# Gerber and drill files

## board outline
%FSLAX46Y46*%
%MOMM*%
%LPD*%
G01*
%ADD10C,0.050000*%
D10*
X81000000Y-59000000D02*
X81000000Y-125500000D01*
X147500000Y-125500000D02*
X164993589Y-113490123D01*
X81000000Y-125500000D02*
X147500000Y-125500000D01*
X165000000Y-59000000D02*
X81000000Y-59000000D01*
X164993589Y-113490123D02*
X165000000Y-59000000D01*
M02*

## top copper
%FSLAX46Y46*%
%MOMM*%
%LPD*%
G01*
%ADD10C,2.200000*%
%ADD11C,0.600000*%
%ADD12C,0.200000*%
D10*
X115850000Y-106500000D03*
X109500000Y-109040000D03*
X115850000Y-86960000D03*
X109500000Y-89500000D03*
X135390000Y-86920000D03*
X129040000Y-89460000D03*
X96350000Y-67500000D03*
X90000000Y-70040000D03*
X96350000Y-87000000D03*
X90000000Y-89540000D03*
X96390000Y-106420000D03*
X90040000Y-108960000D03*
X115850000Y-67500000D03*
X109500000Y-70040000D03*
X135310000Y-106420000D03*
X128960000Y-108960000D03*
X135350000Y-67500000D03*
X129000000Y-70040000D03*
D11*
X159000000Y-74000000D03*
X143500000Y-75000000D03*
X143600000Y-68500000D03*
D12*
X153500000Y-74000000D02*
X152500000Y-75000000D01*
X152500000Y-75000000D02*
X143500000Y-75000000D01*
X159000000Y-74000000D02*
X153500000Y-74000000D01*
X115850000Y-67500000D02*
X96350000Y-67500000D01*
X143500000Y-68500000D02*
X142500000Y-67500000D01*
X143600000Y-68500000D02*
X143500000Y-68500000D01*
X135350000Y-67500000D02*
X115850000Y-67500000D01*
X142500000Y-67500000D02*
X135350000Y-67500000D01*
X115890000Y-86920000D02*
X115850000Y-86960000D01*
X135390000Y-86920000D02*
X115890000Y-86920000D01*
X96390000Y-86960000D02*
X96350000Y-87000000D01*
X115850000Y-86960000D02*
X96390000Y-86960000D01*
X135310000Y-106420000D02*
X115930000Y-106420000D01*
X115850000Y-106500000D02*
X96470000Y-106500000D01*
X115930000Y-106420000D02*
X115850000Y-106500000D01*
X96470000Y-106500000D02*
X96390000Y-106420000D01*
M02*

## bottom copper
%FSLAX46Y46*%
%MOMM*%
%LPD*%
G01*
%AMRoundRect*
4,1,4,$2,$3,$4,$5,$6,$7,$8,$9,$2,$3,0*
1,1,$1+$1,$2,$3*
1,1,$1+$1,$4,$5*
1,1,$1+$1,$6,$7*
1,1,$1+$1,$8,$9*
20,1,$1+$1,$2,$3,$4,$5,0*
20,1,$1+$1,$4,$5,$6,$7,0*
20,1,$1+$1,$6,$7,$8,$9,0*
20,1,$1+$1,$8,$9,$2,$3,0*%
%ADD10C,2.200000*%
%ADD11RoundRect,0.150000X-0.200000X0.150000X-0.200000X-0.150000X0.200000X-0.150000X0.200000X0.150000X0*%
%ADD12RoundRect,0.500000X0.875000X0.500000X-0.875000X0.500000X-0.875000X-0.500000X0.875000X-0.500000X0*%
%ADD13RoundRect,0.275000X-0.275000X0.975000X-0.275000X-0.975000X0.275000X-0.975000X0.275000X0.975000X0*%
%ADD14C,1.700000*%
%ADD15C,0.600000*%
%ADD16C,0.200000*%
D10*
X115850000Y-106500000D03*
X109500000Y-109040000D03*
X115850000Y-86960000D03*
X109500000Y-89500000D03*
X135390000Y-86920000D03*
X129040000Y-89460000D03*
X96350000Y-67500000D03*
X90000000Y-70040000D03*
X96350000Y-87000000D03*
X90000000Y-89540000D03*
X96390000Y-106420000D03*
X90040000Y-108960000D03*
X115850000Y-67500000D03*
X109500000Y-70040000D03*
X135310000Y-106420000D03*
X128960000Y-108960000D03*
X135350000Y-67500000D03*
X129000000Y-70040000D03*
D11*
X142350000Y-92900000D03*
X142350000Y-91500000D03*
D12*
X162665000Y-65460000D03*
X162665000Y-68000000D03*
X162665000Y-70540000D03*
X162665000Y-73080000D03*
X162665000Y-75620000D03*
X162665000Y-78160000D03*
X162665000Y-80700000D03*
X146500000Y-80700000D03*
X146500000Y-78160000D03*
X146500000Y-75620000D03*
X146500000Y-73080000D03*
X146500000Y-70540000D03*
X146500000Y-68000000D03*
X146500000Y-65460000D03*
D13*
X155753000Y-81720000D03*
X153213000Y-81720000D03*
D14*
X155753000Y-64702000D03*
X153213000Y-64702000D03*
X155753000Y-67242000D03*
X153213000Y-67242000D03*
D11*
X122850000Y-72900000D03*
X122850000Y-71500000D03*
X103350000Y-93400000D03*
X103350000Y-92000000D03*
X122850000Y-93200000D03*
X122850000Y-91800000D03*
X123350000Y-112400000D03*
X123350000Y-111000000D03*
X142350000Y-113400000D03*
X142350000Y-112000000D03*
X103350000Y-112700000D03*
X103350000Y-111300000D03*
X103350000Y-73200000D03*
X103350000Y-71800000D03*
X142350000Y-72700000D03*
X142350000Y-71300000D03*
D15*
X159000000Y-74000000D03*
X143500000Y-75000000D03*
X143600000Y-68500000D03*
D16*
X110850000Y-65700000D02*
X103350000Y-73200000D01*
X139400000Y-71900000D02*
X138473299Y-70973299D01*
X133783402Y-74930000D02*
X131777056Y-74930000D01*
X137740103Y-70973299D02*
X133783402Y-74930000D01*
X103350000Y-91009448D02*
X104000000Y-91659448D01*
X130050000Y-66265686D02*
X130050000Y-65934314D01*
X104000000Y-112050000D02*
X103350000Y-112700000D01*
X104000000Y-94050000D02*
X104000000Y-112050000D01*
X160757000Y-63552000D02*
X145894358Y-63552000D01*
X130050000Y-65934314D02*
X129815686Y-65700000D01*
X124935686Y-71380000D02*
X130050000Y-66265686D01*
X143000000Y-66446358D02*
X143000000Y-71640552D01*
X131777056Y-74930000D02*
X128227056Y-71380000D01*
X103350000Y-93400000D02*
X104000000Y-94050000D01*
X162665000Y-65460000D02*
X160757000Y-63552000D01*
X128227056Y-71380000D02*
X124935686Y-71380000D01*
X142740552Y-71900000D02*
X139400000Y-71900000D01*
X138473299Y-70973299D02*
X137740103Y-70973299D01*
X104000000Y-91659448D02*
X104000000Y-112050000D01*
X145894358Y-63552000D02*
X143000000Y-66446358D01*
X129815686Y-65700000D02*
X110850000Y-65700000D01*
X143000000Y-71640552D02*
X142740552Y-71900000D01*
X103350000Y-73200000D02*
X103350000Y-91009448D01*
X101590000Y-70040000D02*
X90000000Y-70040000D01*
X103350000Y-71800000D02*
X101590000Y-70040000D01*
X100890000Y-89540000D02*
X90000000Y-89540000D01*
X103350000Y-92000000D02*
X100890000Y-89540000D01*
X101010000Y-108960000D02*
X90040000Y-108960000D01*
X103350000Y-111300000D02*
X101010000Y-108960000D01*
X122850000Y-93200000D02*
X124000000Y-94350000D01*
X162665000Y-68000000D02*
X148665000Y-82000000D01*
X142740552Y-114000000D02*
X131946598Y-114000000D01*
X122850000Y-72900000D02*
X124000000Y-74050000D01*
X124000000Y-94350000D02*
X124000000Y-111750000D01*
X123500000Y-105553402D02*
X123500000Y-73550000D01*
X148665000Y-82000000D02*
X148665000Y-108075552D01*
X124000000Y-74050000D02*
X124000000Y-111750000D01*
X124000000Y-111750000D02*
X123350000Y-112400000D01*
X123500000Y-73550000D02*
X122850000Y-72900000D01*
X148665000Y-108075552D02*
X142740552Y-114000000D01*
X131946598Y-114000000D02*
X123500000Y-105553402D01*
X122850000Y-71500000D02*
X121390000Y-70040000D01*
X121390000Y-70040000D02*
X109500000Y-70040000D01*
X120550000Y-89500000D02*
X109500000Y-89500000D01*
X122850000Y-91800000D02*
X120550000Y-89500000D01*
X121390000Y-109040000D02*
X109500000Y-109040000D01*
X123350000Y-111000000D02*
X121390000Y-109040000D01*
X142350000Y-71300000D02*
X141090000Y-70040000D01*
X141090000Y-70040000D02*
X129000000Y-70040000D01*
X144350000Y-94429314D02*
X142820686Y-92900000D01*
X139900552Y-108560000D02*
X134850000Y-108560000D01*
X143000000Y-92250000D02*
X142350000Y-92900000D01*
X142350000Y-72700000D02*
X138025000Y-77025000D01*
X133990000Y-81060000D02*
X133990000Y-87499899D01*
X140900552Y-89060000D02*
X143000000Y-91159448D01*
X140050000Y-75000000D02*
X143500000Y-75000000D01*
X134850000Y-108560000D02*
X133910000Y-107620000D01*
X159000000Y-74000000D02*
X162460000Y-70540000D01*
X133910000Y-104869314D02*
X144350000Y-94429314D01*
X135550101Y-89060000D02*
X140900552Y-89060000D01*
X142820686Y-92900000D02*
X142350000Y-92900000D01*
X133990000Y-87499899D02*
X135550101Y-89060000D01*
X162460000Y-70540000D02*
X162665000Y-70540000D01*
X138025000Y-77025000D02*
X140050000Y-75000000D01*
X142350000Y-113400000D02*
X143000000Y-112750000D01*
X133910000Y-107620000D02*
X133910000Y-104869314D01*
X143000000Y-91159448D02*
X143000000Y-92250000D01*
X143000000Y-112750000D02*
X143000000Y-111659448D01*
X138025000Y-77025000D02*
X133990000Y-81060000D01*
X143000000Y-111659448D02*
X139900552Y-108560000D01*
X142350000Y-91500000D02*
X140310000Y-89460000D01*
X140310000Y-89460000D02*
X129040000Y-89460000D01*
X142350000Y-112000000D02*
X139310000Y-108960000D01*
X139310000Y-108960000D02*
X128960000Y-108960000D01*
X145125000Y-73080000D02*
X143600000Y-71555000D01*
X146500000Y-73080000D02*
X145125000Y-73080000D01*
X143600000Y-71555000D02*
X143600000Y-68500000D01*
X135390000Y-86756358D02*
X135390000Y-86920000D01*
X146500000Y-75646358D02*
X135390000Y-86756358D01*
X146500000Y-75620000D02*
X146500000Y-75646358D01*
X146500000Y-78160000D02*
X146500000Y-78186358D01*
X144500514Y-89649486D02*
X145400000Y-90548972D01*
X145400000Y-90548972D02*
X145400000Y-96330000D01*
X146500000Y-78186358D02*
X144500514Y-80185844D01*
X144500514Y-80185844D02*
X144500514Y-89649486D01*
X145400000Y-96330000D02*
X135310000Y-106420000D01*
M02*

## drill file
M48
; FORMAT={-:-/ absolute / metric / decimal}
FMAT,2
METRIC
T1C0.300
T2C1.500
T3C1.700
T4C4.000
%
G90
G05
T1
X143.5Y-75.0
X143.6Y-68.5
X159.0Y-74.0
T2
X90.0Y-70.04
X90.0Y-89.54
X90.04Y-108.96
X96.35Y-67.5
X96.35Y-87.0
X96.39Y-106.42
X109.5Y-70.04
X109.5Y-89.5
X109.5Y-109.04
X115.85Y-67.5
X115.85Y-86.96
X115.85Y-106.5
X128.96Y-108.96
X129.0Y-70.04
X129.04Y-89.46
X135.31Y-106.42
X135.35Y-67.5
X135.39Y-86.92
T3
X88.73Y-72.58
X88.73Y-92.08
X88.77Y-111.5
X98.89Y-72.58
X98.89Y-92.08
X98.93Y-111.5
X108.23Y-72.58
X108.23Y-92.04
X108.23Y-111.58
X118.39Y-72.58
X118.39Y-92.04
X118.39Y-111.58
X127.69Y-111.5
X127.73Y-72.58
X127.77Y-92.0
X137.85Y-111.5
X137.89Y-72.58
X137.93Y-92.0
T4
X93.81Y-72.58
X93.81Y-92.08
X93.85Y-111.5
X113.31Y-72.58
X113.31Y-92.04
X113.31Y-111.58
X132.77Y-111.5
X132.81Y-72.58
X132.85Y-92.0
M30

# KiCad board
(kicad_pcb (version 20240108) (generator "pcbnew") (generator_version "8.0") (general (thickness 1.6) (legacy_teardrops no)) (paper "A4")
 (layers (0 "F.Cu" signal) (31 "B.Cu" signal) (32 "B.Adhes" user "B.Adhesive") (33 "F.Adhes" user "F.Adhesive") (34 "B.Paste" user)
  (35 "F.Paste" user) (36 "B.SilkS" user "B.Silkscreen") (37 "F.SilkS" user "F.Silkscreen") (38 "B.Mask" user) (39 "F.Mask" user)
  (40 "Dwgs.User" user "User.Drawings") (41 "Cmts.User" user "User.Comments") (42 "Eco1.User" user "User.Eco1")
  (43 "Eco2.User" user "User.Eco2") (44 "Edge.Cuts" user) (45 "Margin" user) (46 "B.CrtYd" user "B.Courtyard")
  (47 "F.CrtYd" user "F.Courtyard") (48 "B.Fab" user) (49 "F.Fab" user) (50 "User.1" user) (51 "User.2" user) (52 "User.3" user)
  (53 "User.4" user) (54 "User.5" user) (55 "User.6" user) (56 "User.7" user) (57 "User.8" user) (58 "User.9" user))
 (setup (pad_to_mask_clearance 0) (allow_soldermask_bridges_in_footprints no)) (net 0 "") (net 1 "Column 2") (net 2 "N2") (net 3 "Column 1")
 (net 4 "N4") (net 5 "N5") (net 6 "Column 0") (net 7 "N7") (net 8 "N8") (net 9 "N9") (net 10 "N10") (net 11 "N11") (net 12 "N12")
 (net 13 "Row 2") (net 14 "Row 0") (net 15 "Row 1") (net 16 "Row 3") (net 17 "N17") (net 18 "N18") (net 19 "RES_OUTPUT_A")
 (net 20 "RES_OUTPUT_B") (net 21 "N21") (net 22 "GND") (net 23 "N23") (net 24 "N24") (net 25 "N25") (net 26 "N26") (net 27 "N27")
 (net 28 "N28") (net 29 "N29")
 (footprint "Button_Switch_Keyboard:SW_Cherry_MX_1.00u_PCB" (layer "F.Cu") (at 115.85 106.5)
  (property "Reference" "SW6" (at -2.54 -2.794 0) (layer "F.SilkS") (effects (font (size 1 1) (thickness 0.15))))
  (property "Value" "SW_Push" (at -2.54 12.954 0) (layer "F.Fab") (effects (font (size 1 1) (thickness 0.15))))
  (pad "" np_thru_hole circle (at -7.62 5.08) (size 1.7 1.7) (drill 1.7) (layers "*.Cu" "*.Mask"))
  (pad "" np_thru_hole circle (at -2.54 5.08) (size 4 4) (drill 4) (layers "*.Cu" "*.Mask"))
  (pad "" np_thru_hole circle (at 2.54 5.08) (size 1.7 1.7) (drill 1.7) (layers "*.Cu" "*.Mask"))
  (pad "1" thru_hole circle (at 0 0) (size 2.2 2.2) (drill 1.5) (layers "*.Cu" "*.Mask") (remove_unused_layers no) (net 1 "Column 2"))
  (pad "2" thru_hole circle (at -6.35 2.54) (size 2.2 2.2) (drill 1.5) (layers "*.Cu" "*.Mask") (remove_unused_layers no) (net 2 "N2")))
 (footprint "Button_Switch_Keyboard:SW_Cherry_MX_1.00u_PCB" (layer "F.Cu") (at 115.85 86.96)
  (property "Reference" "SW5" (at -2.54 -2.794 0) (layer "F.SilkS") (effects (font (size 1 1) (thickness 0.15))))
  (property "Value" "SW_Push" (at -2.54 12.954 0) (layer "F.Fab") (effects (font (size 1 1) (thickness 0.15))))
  (pad "" np_thru_hole circle (at -7.62 5.08) (size 1.7 1.7) (drill 1.7) (layers "*.Cu" "*.Mask"))
  (pad "" np_thru_hole circle (at -2.54 5.08) (size 4 4) (drill 4) (layers "*.Cu" "*.Mask"))
  (pad "" np_thru_hole circle (at 2.54 5.08) (size 1.7 1.7) (drill 1.7) (layers "*.Cu" "*.Mask"))
  (pad "1" thru_hole circle (at 0 0) (size 2.2 2.2) (drill 1.5) (layers "*.Cu" "*.Mask") (remove_unused_layers no) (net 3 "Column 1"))
  (pad "2" thru_hole circle (at -6.35 2.54) (size 2.2 2.2) (drill 1.5) (layers "*.Cu" "*.Mask") (remove_unused_layers no) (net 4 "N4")))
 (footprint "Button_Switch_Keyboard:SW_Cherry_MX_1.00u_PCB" (layer "F.Cu") (at 135.39 86.92)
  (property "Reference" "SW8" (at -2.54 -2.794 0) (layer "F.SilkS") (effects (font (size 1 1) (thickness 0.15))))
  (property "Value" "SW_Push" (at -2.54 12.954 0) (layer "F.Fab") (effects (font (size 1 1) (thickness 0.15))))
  (pad "" np_thru_hole circle (at -7.62 5.08) (size 1.7 1.7) (drill 1.7) (layers "*.Cu" "*.Mask"))
  (pad "" np_thru_hole circle (at -2.54 5.08) (size 4 4) (drill 4) (layers "*.Cu" "*.Mask"))
  (pad "" np_thru_hole circle (at 2.54 5.08) (size 1.7 1.7) (drill 1.7) (layers "*.Cu" "*.Mask"))
  (pad "1" thru_hole circle (at 0 0) (size 2.2 2.2) (drill 1.5) (layers "*.Cu" "*.Mask") (remove_unused_layers no) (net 3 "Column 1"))
  (pad "2" thru_hole circle (at -6.35 2.54) (size 2.2 2.2) (drill 1.5) (layers "*.Cu" "*.Mask") (remove_unused_layers no) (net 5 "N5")))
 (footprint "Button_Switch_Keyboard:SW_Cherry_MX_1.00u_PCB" (layer "F.Cu") (at 96.35 67.5)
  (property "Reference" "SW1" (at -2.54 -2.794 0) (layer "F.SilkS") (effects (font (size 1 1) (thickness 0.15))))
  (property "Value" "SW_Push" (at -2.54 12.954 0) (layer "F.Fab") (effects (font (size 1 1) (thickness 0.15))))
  (pad "" np_thru_hole circle (at -7.62 5.08) (size 1.7 1.7) (drill 1.7) (layers "*.Cu" "*.Mask"))
  (pad "" np_thru_hole circle (at -2.54 5.08) (size 4 4) (drill 4) (layers "*.Cu" "*.Mask"))
  (pad "" np_thru_hole circle (at 2.54 5.08) (size 1.7 1.7) (drill 1.7) (layers "*.Cu" "*.Mask"))
  (pad "1" thru_hole circle (at 0 0) (size 2.2 2.2) (drill 1.5) (layers "*.Cu" "*.Mask") (remove_unused_layers no) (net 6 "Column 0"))
  (pad "2" thru_hole circle (at -6.35 2.54) (size 2.2 2.2) (drill 1.5) (layers "*.Cu" "*.Mask") (remove_unused_layers no) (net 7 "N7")))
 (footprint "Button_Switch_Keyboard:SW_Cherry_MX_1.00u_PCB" (layer "F.Cu") (at 96.35 87)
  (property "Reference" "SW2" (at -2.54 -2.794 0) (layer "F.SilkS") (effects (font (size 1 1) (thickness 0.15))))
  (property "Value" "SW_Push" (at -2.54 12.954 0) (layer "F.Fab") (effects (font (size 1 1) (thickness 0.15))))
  (pad "" np_thru_hole circle (at -7.62 5.08) (size 1.7 1.7) (drill 1.7) (layers "*.Cu" "*.Mask"))
  (pad "" np_thru_hole circle (at -2.54 5.08) (size 4 4) (drill 4) (layers "*.Cu" "*.Mask"))
  (pad "" np_thru_hole circle (at 2.54 5.08) (size 1.7 1.7) (drill 1.7) (layers "*.Cu" "*.Mask"))
  (pad "1" thru_hole circle (at 0 0) (size 2.2 2.2) (drill 1.5) (layers "*.Cu" "*.Mask") (remove_unused_layers no) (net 3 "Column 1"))
  (pad "2" thru_hole circle (at -6.35 2.54) (size 2.2 2.2) (drill 1.5) (layers "*.Cu" "*.Mask") (remove_unused_layers no) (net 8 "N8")))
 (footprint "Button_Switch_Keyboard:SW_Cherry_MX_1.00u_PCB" (layer "F.Cu") (at 96.39 106.42)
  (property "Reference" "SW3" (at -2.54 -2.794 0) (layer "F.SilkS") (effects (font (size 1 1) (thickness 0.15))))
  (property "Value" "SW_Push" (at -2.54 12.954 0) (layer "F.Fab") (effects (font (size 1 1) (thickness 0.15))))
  (pad "" np_thru_hole circle (at -7.62 5.08) (size 1.7 1.7) (drill 1.7) (layers "*.Cu" "*.Mask"))
  (pad "" np_thru_hole circle (at -2.54 5.08) (size 4 4) (drill 4) (layers "*.Cu" "*.Mask"))
  (pad "" np_thru_hole circle (at 2.54 5.08) (size 1.7 1.7) (drill 1.7) (layers "*.Cu" "*.Mask"))
  (pad "1" thru_hole circle (at 0 0) (size 2.2 2.2) (drill 1.5) (layers "*.Cu" "*.Mask") (remove_unused_layers no) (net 1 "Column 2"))
  (pad "2" thru_hole circle (at -6.35 2.54) (size 2.2 2.2) (drill 1.5) (layers "*.Cu" "*.Mask") (remove_unused_layers no) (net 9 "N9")))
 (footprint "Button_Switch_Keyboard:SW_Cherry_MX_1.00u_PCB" (layer "F.Cu") (at 115.85 67.5)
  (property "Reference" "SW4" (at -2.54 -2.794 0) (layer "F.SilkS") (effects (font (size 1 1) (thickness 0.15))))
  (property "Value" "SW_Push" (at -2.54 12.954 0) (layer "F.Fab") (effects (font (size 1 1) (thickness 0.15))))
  (pad "" np_thru_hole circle (at -7.62 5.08) (size 1.7 1.7) (drill 1.7) (layers "*.Cu" "*.Mask"))
  (pad "" np_thru_hole circle (at -2.54 5.08) (size 4 4) (drill 4) (layers "*.Cu" "*.Mask"))
  (pad "" np_thru_hole circle (at 2.54 5.08) (size 1.7 1.7) (drill 1.7) (layers "*.Cu" "*.Mask"))
  (pad "1" thru_hole circle (at 0 0) (size 2.2 2.2) (drill 1.5) (layers "*.Cu" "*.Mask") (remove_unused_layers no) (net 6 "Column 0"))
  (pad "2" thru_hole circle (at -6.35 2.54) (size 2.2 2.2) (drill 1.5) (layers "*.Cu" "*.Mask") (remove_unused_layers no) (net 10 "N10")))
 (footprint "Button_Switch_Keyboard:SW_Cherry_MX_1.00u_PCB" (layer "F.Cu") (at 135.31 106.42)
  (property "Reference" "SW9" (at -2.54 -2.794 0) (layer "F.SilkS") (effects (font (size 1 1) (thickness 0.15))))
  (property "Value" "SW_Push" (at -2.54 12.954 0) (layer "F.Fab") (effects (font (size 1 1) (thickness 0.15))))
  (pad "" np_thru_hole circle (at -7.62 5.08) (size 1.7 1.7) (drill 1.7) (layers "*.Cu" "*.Mask"))
  (pad "" np_thru_hole circle (at -2.54 5.08) (size 4 4) (drill 4) (layers "*.Cu" "*.Mask"))
  (pad "" np_thru_hole circle (at 2.54 5.08) (size 1.7 1.7) (drill 1.7) (layers "*.Cu" "*.Mask"))
  (pad "1" thru_hole circle (at 0 0) (size 2.2 2.2) (drill 1.5) (layers "*.Cu" "*.Mask") (remove_unused_layers no) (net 1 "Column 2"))
  (pad "2" thru_hole circle (at -6.35 2.54) (size 2.2 2.2) (drill 1.5) (layers "*.Cu" "*.Mask") (remove_unused_layers no) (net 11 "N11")))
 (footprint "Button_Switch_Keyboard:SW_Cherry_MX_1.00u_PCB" (layer "F.Cu") (at 135.35 67.5)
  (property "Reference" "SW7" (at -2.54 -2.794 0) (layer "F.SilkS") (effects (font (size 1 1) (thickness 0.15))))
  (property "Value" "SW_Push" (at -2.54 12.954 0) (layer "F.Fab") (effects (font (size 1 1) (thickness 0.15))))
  (pad "" np_thru_hole circle (at -7.62 5.08) (size 1.7 1.7) (drill 1.7) (layers "*.Cu" "*.Mask"))
  (pad "" np_thru_hole circle (at -2.54 5.08) (size 4 4) (drill 4) (layers "*.Cu" "*.Mask"))
  (pad "" np_thru_hole circle (at 2.54 5.08) (size 1.7 1.7) (drill 1.7) (layers "*.Cu" "*.Mask"))
  (pad "1" thru_hole circle (at 0 0) (size 2.2 2.2) (drill 1.5) (layers "*.Cu" "*.Mask") (remove_unused_layers no) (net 6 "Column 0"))
  (pad "2" thru_hole circle (at -6.35 2.54) (size 2.2 2.2) (drill 1.5) (layers "*.Cu" "*.Mask") (remove_unused_layers no) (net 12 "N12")))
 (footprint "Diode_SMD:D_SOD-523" (layer "B.Cu") (at 142.35 92.2 90)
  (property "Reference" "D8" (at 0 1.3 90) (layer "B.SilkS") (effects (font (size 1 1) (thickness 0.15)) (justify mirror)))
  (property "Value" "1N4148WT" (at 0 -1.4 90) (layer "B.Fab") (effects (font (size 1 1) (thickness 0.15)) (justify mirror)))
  (pad "1" smd roundrect (at -0.7 0 270) (size 0.6 0.7) (layers "B.Cu" "B.Paste" "B.Mask") (roundrect_rratio 0.25) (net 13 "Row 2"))
  (pad "2" smd roundrect (at 0.7 0 270) (size 0.6 0.7) (layers "B.Cu" "B.Paste" "B.Mask") (roundrect_rratio 0.25) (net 5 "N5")))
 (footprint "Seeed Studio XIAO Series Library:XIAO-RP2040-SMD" (layer "B.Cu") (at 154.665 73.08 180)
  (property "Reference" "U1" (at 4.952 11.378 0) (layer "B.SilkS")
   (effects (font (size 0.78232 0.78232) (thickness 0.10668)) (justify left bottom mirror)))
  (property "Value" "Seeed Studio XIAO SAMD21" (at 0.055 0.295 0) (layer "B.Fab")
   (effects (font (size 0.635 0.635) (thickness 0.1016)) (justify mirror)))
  (pad "1" smd roundrect (at -8 7.62 180) (size 2.75 2) (layers "B.Cu" "B.Paste" "B.Mask") (roundrect_rratio 0.25) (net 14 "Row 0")
   (solder_mask_margin 0.0508) (thermal_bridge_angle 45))
  (pad "2" smd roundrect (at -8 5.08 180) (size 2.75 2) (layers "B.Cu" "B.Paste" "B.Mask") (roundrect_rratio 0.25) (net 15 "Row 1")
   (solder_mask_margin 0.0508) (thermal_bridge_angle 45))
  (pad "3" smd roundrect (at -8 2.54 180) (size 2.75 2) (layers "B.Cu" "B.Paste" "B.Mask") (roundrect_rratio 0.25) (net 13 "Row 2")
   (solder_mask_margin 0.0508) (thermal_bridge_angle 45))
  (pad "4" smd roundrect (at -8 0 180) (size 2.75 2) (layers "B.Cu" "B.Paste" "B.Mask") (roundrect_rratio 0.25) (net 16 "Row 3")
   (solder_mask_margin 0.0508) (thermal_bridge_angle 45))
  (pad "5" smd roundrect (at -8 -2.54 180) (size 2.75 2) (layers "B.Cu" "B.Paste" "B.Mask") (roundrect_rratio 0.25) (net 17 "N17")
   (solder_mask_margin 0.0508) (thermal_bridge_angle 45))
  (pad "6" smd roundrect (at -8 -5.08 180) (size 2.75 2) (layers "B.Cu" "B.Paste" "B.Mask") (roundrect_rratio 0.25) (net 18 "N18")
   (solder_mask_margin 0.0508) (thermal_bridge_angle 45))
  (pad "7" smd roundrect (at -8 -7.62 180) (size 2.75 2) (layers "B.Cu" "B.Paste" "B.Mask") (roundrect_rratio 0.25) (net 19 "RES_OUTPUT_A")
   (solder_mask_margin 0.0508) (thermal_bridge_angle 45))
  (pad "8" smd roundrect (at 8.165 -7.62 180) (size 2.75 2) (layers "B.Cu" "B.Paste" "B.Mask") (roundrect_rratio 0.25)
   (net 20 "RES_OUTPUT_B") (solder_mask_margin 0.0508) (thermal_bridge_angle 45))
  (pad "9" smd roundrect (at 8.165 -5.08 180) (size 2.75 2) (layers "B.Cu" "B.Paste" "B.Mask") (roundrect_rratio 0.25) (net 1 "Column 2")
   (solder_mask_margin 0.0508) (thermal_bridge_angle 45))
  (pad "10" smd roundrect (at 8.165 -2.54 180) (size 2.75 2) (layers "B.Cu" "B.Paste" "B.Mask") (roundrect_rratio 0.25) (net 3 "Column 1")
   (solder_mask_margin 0.0508) (thermal_bridge_angle 45))
  (pad "11" smd roundrect (at 8.165 0 180) (size 2.75 2) (layers "B.Cu" "B.Paste" "B.Mask") (roundrect_rratio 0.25) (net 6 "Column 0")
   (solder_mask_margin 0.0508) (thermal_bridge_angle 45))
  (pad "12" smd roundrect (at 8.165 2.54 180) (size 2.75 2) (layers "B.Cu" "B.Paste" "B.Mask") (roundrect_rratio 0.25) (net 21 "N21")
   (solder_mask_margin 0.0508) (thermal_bridge_angle 45))
  (pad "13" smd roundrect (at 8.165 5.08 180) (size 2.75 2) (layers "B.Cu" "B.Paste" "B.Mask") (roundrect_rratio 0.25) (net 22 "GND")
   (solder_mask_margin 0.0508) (thermal_bridge_angle 45))
  (pad "14" smd roundrect (at 8.165 7.62 180) (size 2.75 2) (layers "B.Cu" "B.Paste" "B.Mask") (roundrect_rratio 0.25) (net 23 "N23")
   (solder_mask_margin 0.0508) (thermal_bridge_angle 45))
  (pad "15" smd roundrect (at -1.088 -8.64 270) (size 2.5 1.1) (layers "B.Cu" "B.Paste" "B.Mask") (roundrect_rratio 0.25) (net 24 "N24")
   (thermal_bridge_angle 45))
  (pad "16" smd roundrect (at 1.452 -8.64 270) (size 2.5 1.1) (layers "B.Cu" "B.Paste" "B.Mask") (roundrect_rratio 0.25) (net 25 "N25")
   (thermal_bridge_angle 45))
  (pad "17" smd circle (at -1.088 8.378 180) (size 1.7 1.7) (layers "B.Cu" "B.Paste" "B.Mask") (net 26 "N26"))
  (pad "18" smd circle (at 1.452 8.378 180) (size 1.7 1.7) (layers "B.Cu" "B.Paste" "B.Mask") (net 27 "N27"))
  (pad "19" smd circle (at -1.088 5.838 180) (size 1.7 1.7) (layers "B.Cu" "B.Paste" "B.Mask") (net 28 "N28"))
  (pad "20" smd circle (at 1.452 5.838 180) (size 1.7 1.7) (layers "B.Cu" "B.Paste" "B.Mask") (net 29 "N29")))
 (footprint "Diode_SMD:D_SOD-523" (layer "B.Cu") (at 122.85 72.2 90)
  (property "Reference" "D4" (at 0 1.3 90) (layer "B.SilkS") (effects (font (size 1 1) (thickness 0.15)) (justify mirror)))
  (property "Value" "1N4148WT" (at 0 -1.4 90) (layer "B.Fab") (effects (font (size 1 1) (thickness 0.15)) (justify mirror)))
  (pad "1" smd roundrect (at -0.7 0 270) (size 0.6 0.7) (layers "B.Cu" "B.Paste" "B.Mask") (roundrect_rratio 0.25) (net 15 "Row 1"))
  (pad "2" smd roundrect (at 0.7 0 270) (size 0.6 0.7) (layers "B.Cu" "B.Paste" "B.Mask") (roundrect_rratio 0.25) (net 10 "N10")))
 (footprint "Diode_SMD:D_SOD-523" (layer "B.Cu") (at 103.35 92.7 90)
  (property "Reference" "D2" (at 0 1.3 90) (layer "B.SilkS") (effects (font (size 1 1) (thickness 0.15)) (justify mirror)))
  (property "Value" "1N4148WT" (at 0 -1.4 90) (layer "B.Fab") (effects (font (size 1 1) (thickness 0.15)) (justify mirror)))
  (pad "1" smd roundrect (at -0.7 0 270) (size 0.6 0.7) (layers "B.Cu" "B.Paste" "B.Mask") (roundrect_rratio 0.25) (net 14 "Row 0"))
  (pad "2" smd roundrect (at 0.7 0 270) (size 0.6 0.7) (layers "B.Cu" "B.Paste" "B.Mask") (roundrect_rratio 0.25) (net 8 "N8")))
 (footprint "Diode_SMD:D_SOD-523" (layer "B.Cu") (at 122.85 92.5 90)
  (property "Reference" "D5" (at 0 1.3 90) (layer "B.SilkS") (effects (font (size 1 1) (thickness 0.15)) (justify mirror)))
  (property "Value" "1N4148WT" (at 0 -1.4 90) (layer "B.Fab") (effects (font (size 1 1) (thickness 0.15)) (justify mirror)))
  (pad "1" smd roundrect (at -0.7 0 270) (size 0.6 0.7) (layers "B.Cu" "B.Paste" "B.Mask") (roundrect_rratio 0.25) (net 15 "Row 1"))
  (pad "2" smd roundrect (at 0.7 0 270) (size 0.6 0.7) (layers "B.Cu" "B.Paste" "B.Mask") (roundrect_rratio 0.25) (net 4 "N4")))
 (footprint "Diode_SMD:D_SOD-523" (layer "B.Cu") (at 123.35 111.7 90)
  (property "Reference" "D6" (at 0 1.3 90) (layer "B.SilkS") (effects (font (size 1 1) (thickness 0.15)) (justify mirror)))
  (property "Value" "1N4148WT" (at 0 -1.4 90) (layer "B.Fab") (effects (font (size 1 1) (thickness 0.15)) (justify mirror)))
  (pad "1" smd roundrect (at -0.7 0 270) (size 0.6 0.7) (layers "B.Cu" "B.Paste" "B.Mask") (roundrect_rratio 0.25) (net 15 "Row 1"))
  (pad "2" smd roundrect (at 0.7 0 270) (size 0.6 0.7) (layers "B.Cu" "B.Paste" "B.Mask") (roundrect_rratio 0.25) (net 2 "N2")))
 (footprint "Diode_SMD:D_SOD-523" (layer "B.Cu") (at 142.35 112.7 90)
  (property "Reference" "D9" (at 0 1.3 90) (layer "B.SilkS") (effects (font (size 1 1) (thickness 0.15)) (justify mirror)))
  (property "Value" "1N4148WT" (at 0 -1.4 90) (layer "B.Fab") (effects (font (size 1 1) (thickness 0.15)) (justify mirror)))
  (pad "1" smd roundrect (at -0.7 0 270) (size 0.6 0.7) (layers "B.Cu" "B.Paste" "B.Mask") (roundrect_rratio 0.25) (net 13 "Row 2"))
  (pad "2" smd roundrect (at 0.7 0 270) (size 0.6 0.7) (layers "B.Cu" "B.Paste" "B.Mask") (roundrect_rratio 0.25) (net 11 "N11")))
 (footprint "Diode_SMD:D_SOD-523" (layer "B.Cu") (at 103.35 112 90)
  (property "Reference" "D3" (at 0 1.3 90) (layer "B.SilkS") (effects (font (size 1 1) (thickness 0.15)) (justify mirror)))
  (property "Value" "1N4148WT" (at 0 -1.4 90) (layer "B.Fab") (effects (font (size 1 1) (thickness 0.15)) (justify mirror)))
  (pad "1" smd roundrect (at -0.7 0 270) (size 0.6 0.7) (layers "B.Cu" "B.Paste" "B.Mask") (roundrect_rratio 0.25) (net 14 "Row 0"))
  (pad "2" smd roundrect (at 0.7 0 270) (size 0.6 0.7) (layers "B.Cu" "B.Paste" "B.Mask") (roundrect_rratio 0.25) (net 9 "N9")))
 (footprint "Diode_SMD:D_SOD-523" (layer "B.Cu") (at 103.35 72.5 90)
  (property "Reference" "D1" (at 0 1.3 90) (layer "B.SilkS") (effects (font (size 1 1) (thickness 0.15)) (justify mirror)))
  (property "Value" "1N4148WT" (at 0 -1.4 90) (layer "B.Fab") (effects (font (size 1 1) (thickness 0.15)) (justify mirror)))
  (pad "1" smd roundrect (at -0.7 0 270) (size 0.6 0.7) (layers "B.Cu" "B.Paste" "B.Mask") (roundrect_rratio 0.25) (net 14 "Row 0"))
  (pad "2" smd roundrect (at 0.7 0 270) (size 0.6 0.7) (layers "B.Cu" "B.Paste" "B.Mask") (roundrect_rratio 0.25) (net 7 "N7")))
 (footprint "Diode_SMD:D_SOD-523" (layer "B.Cu") (at 142.35 72 90)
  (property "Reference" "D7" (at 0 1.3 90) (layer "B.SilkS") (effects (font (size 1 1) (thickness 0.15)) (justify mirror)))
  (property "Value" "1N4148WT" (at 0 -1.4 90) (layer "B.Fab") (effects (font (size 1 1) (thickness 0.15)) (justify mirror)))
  (pad "1" smd roundrect (at -0.7 0 270) (size 0.6 0.7) (layers "B.Cu" "B.Paste" "B.Mask") (roundrect_rratio 0.25) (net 13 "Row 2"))
  (pad "2" smd roundrect (at 0.7 0 270) (size 0.6 0.7) (layers "B.Cu" "B.Paste" "B.Mask") (roundrect_rratio 0.25) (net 12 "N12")))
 (gr_line (start 81 59) (end 81 125.5) (stroke (width 0.05) (type default)) (layer "Edge.Cuts"))
 (gr_line (start 147.5 125.5) (end 164.993589 113.490123) (stroke (width 0.05) (type default)) (layer "Edge.Cuts"))
 (gr_line (start 81 125.5) (end 147.5 125.5) (stroke (width 0.05) (type default)) (layer "Edge.Cuts"))
 (gr_line (start 165 59) (end 81 59) (stroke (width 0.05) (type default)) (layer "Edge.Cuts"))
 (gr_line (start 164.993589 113.490123) (end 165 59) (stroke (width 0.05) (type default)) (layer "Edge.Cuts"))
 (segment (start 110.85 65.7) (end 103.35 73.2) (width 0.2) (layer "B.Cu") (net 14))
 (segment (start 139.4 71.9) (end 138.473299 70.973299) (width 0.2) (layer "B.Cu") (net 14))
 (segment (start 133.783402 74.93) (end 131.777056 74.93) (width 0.2) (layer "B.Cu") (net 14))
 (segment (start 137.740103 70.973299) (end 133.783402 74.93) (width 0.2) (layer "B.Cu") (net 14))
 (segment (start 103.35 91.009448) (end 104 91.659448) (width 0.2) (layer "B.Cu") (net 14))
 (segment (start 130.05 66.265686) (end 130.05 65.934314) (width 0.2) (layer "B.Cu") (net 14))
 (segment (start 104 112.05) (end 103.35 112.7) (width 0.2) (layer "B.Cu") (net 14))
 (segment (start 104 94.05) (end 104 112.05) (width 0.2) (layer "B.Cu") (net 14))
 (segment (start 160.757 63.552) (end 145.894358 63.552) (width 0.2) (layer "B.Cu") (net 14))
 (segment (start 130.05 65.934314) (end 129.815686 65.7) (width 0.2) (layer "B.Cu") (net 14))
 (segment (start 124.935686 71.38) (end 130.05 66.265686) (width 0.2) (layer "B.Cu") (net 14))
 (segment (start 143 66.446358) (end 143 71.640552) (width 0.2) (layer "B.Cu") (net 14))
 (segment (start 131.777056 74.93) (end 128.227056 71.38) (width 0.2) (layer "B.Cu") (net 14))
 (segment (start 103.35 93.4) (end 104 94.05) (width 0.2) (layer "B.Cu") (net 14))
 (segment (start 162.665 65.46) (end 160.757 63.552) (width 0.2) (layer "B.Cu") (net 14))
 (segment (start 128.227056 71.38) (end 124.935686 71.38) (width 0.2) (layer "B.Cu") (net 14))
 (segment (start 142.740552 71.9) (end 139.4 71.9) (width 0.2) (layer "B.Cu") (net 14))
 (segment (start 138.473299 70.973299) (end 137.740103 70.973299) (width 0.2) (layer "B.Cu") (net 14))
 (segment (start 104 91.659448) (end 104 112.05) (width 0.2) (layer "B.Cu") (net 14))
 (segment (start 145.894358 63.552) (end 143 66.446358) (width 0.2) (layer "B.Cu") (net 14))
 (segment (start 129.815686 65.7) (end 110.85 65.7) (width 0.2) (layer "B.Cu") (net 14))
 (segment (start 143 71.640552) (end 142.740552 71.9) (width 0.2) (layer "B.Cu") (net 14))
 (segment (start 103.35 73.2) (end 103.35 91.009448) (width 0.2) (layer "B.Cu") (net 14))
 (segment (start 101.59 70.04) (end 90 70.04) (width 0.2) (layer "B.Cu") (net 7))
 (segment (start 103.35 71.8) (end 101.59 70.04) (width 0.2) (layer "B.Cu") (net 7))
 (segment (start 100.89 89.54) (end 90 89.54) (width 0.2) (layer "B.Cu") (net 8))
 (segment (start 103.35 92) (end 100.89 89.54) (width 0.2) (layer "B.Cu") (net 8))
 (segment (start 101.01 108.96) (end 90.04 108.96) (width 0.2) (layer "B.Cu") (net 9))
 (segment (start 103.35 111.3) (end 101.01 108.96) (width 0.2) (layer "B.Cu") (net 9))
 (segment (start 122.85 93.2) (end 124 94.35) (width 0.2) (layer "B.Cu") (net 15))
 (segment (start 162.665 68) (end 148.665 82) (width 0.2) (layer "B.Cu") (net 15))
 (segment (start 142.740552 114) (end 131.946598 114) (width 0.2) (layer "B.Cu") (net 15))
 (segment (start 122.85 72.9) (end 124 74.05) (width 0.2) (layer "B.Cu") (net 15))
 (segment (start 124 94.35) (end 124 111.75) (width 0.2) (layer "B.Cu") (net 15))
 (segment (start 123.5 105.553402) (end 123.5 73.55) (width 0.2) (layer "B.Cu") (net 15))
 (segment (start 148.665 82) (end 148.665 108.075552) (width 0.2) (layer "B.Cu") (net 15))
 (segment (start 124 74.05) (end 124 111.75) (width 0.2) (layer "B.Cu") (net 15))
 (segment (start 124 111.75) (end 123.35 112.4) (width 0.2) (layer "B.Cu") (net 15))
 (segment (start 123.5 73.55) (end 122.85 72.9) (width 0.2) (layer "B.Cu") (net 15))
 (segment (start 148.665 108.075552) (end 142.740552 114) (width 0.2) (layer "B.Cu") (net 15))
 (segment (start 131.946598 114) (end 123.5 105.553402) (width 0.2) (layer "B.Cu") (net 15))
 (segment (start 122.85 71.5) (end 121.39 70.04) (width 0.2) (layer "B.Cu") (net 10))
 (segment (start 121.39 70.04) (end 109.5 70.04) (width 0.2) (layer "B.Cu") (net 10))
 (segment (start 120.55 89.5) (end 109.5 89.5) (width 0.2) (layer "B.Cu") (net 4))
 (segment (start 122.85 91.8) (end 120.55 89.5) (width 0.2) (layer "B.Cu") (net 4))
 (segment (start 121.39 109.04) (end 109.5 109.04) (width 0.2) (layer "B.Cu") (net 2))
 (segment (start 123.35 111) (end 121.39 109.04) (width 0.2) (layer "B.Cu") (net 2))
 (segment (start 142.35 71.3) (end 141.09 70.04) (width 0.2) (layer "B.Cu") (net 12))
 (segment (start 141.09 70.04) (end 129 70.04) (width 0.2) (layer "B.Cu") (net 12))
 (segment (start 153.5 74) (end 152.5 75) (width 0.2) (layer "F.Cu") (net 13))
 (segment (start 152.5 75) (end 143.5 75) (width 0.2) (layer "F.Cu") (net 13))
 (segment (start 159 74) (end 153.5 74) (width 0.2) (layer "F.Cu") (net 13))
 (via (at 159 74) (size 0.6) (drill 0.3) (layers "F.Cu" "B.Cu") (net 13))
 (via (at 143.5 75) (size 0.6) (drill 0.3) (layers "F.Cu" "B.Cu") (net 13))
 (segment (start 144.35 94.429314) (end 142.820686 92.9) (width 0.2) (layer "B.Cu") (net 13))
 (segment (start 139.900552 108.56) (end 134.85 108.56) (width 0.2) (layer "B.Cu") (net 13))
 (segment (start 143 92.25) (end 142.35 92.9) (width 0.2) (layer "B.Cu") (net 13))
 (segment (start 142.35 72.7) (end 138.025 77.025) (width 0.2) (layer "B.Cu") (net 13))
 (segment (start 133.99 81.06) (end 133.99 87.499899) (width 0.2) (layer "B.Cu") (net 13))
 (segment (start 140.900552 89.06) (end 143 91.159448) (width 0.2) (layer "B.Cu") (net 13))
 (segment (start 140.05 75) (end 143.5 75) (width 0.2) (layer "B.Cu") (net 13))
 (segment (start 134.85 108.56) (end 133.91 107.62) (width 0.2) (layer "B.Cu") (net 13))
 (segment (start 159 74) (end 162.46 70.54) (width 0.2) (layer "B.Cu") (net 13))
 (segment (start 133.91 104.869314) (end 144.35 94.429314) (width 0.2) (layer "B.Cu") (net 13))
 (segment (start 135.550101 89.06) (end 140.900552 89.06) (width 0.2) (layer "B.Cu") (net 13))
 (segment (start 142.820686 92.9) (end 142.35 92.9) (width 0.2) (layer "B.Cu") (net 13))
 (segment (start 133.99 87.499899) (end 135.550101 89.06) (width 0.2) (layer "B.Cu") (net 13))
 (segment (start 162.46 70.54) (end 162.665 70.54) (width 0.2) (layer "B.Cu") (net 13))
 (segment (start 138.025 77.025) (end 140.05 75) (width 0.2) (layer "B.Cu") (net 13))
 (segment (start 142.35 113.4) (end 143 112.75) (width 0.2) (layer "B.Cu") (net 13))
 (segment (start 133.91 107.62) (end 133.91 104.869314) (width 0.2) (layer "B.Cu") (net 13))
 (segment (start 143 91.159448) (end 143 92.25) (width 0.2) (layer "B.Cu") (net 13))
 (segment (start 143 112.75) (end 143 111.659448) (width 0.2) (layer "B.Cu") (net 13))
 (segment (start 138.025 77.025) (end 133.99 81.06) (width 0.2) (layer "B.Cu") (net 13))
 (segment (start 143 111.659448) (end 139.900552 108.56) (width 0.2) (layer "B.Cu") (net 13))
 (segment (start 142.35 91.5) (end 140.31 89.46) (width 0.2) (layer "B.Cu") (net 5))
 (segment (start 140.31 89.46) (end 129.04 89.46) (width 0.2) (layer "B.Cu") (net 5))
 (segment (start 142.35 112) (end 139.31 108.96) (width 0.2) (layer "B.Cu") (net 11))
 (segment (start 139.31 108.96) (end 128.96 108.96) (width 0.2) (layer "B.Cu") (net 11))
 (segment (start 115.85 67.5) (end 96.35 67.5) (width 0.2) (layer "F.Cu") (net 6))
 (segment (start 143.5 68.5) (end 142.5 67.5) (width 0.2) (layer "F.Cu") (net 6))
 (segment (start 143.6 68.5) (end 143.5 68.5) (width 0.2) (layer "F.Cu") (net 6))
 (segment (start 135.35 67.5) (end 115.85 67.5) (width 0.2) (layer "F.Cu") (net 6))
 (segment (start 142.5 67.5) (end 135.35 67.5) (width 0.2) (layer "F.Cu") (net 6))
 (via (at 143.6 68.5) (size 0.6) (drill 0.3) (layers "F.Cu" "B.Cu") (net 6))
 (segment (start 145.125 73.08) (end 143.6 71.555) (width 0.2) (layer "B.Cu") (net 6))
 (segment (start 146.5 73.08) (end 145.125 73.08) (width 0.2) (layer "B.Cu") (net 6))
 (segment (start 143.6 71.555) (end 143.6 68.5) (width 0.2) (layer "B.Cu") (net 6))
 (segment (start 115.89 86.92) (end 115.85 86.96) (width 0.2) (layer "F.Cu") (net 3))
 (segment (start 135.39 86.92) (end 115.89 86.92) (width 0.2) (layer "F.Cu") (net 3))
 (segment (start 96.39 86.96) (end 96.35 87) (width 0.2) (layer "F.Cu") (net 3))
 (segment (start 115.85 86.96) (end 96.39 86.96) (width 0.2) (layer "F.Cu") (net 3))
 (segment (start 135.39 86.756358) (end 135.39 86.92) (width 0.2) (layer "B.Cu") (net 3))
 (segment (start 146.5 75.646358) (end 135.39 86.756358) (width 0.2) (layer "B.Cu") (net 3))
 (segment (start 146.5 75.62) (end 146.5 75.646358) (width 0.2) (layer "B.Cu") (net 3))
 (segment (start 135.31 106.42) (end 115.93 106.42) (width 0.2) (layer "F.Cu") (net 1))
 (segment (start 115.85 106.5) (end 96.47 106.5) (width 0.2) (layer "F.Cu") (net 1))
 (segment (start 115.93 106.42) (end 115.85 106.5) (width 0.2) (layer "F.Cu") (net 1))
 (segment (start 96.47 106.5) (end 96.39 106.42) (width 0.2) (layer "F.Cu") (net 1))
 (segment (start 146.5 78.16) (end 146.5 78.186358) (width 0.2) (layer "B.Cu") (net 1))
 (segment (start 144.500514 89.649486) (end 145.4 90.548972) (width 0.2) (layer "B.Cu") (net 1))
 (segment (start 145.4 90.548972) (end 145.4 96.33) (width 0.2) (layer "B.Cu") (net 1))
 (segment (start 146.5 78.186358) (end 144.500514 80.185844) (width 0.2) (layer "B.Cu") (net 1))
 (segment (start 144.500514 80.185844) (end 144.500514 89.649486) (width 0.2) (layer "B.Cu") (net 1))
 (segment (start 145.4 96.33) (end 135.31 106.42) (width 0.2) (layer "B.Cu") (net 1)))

